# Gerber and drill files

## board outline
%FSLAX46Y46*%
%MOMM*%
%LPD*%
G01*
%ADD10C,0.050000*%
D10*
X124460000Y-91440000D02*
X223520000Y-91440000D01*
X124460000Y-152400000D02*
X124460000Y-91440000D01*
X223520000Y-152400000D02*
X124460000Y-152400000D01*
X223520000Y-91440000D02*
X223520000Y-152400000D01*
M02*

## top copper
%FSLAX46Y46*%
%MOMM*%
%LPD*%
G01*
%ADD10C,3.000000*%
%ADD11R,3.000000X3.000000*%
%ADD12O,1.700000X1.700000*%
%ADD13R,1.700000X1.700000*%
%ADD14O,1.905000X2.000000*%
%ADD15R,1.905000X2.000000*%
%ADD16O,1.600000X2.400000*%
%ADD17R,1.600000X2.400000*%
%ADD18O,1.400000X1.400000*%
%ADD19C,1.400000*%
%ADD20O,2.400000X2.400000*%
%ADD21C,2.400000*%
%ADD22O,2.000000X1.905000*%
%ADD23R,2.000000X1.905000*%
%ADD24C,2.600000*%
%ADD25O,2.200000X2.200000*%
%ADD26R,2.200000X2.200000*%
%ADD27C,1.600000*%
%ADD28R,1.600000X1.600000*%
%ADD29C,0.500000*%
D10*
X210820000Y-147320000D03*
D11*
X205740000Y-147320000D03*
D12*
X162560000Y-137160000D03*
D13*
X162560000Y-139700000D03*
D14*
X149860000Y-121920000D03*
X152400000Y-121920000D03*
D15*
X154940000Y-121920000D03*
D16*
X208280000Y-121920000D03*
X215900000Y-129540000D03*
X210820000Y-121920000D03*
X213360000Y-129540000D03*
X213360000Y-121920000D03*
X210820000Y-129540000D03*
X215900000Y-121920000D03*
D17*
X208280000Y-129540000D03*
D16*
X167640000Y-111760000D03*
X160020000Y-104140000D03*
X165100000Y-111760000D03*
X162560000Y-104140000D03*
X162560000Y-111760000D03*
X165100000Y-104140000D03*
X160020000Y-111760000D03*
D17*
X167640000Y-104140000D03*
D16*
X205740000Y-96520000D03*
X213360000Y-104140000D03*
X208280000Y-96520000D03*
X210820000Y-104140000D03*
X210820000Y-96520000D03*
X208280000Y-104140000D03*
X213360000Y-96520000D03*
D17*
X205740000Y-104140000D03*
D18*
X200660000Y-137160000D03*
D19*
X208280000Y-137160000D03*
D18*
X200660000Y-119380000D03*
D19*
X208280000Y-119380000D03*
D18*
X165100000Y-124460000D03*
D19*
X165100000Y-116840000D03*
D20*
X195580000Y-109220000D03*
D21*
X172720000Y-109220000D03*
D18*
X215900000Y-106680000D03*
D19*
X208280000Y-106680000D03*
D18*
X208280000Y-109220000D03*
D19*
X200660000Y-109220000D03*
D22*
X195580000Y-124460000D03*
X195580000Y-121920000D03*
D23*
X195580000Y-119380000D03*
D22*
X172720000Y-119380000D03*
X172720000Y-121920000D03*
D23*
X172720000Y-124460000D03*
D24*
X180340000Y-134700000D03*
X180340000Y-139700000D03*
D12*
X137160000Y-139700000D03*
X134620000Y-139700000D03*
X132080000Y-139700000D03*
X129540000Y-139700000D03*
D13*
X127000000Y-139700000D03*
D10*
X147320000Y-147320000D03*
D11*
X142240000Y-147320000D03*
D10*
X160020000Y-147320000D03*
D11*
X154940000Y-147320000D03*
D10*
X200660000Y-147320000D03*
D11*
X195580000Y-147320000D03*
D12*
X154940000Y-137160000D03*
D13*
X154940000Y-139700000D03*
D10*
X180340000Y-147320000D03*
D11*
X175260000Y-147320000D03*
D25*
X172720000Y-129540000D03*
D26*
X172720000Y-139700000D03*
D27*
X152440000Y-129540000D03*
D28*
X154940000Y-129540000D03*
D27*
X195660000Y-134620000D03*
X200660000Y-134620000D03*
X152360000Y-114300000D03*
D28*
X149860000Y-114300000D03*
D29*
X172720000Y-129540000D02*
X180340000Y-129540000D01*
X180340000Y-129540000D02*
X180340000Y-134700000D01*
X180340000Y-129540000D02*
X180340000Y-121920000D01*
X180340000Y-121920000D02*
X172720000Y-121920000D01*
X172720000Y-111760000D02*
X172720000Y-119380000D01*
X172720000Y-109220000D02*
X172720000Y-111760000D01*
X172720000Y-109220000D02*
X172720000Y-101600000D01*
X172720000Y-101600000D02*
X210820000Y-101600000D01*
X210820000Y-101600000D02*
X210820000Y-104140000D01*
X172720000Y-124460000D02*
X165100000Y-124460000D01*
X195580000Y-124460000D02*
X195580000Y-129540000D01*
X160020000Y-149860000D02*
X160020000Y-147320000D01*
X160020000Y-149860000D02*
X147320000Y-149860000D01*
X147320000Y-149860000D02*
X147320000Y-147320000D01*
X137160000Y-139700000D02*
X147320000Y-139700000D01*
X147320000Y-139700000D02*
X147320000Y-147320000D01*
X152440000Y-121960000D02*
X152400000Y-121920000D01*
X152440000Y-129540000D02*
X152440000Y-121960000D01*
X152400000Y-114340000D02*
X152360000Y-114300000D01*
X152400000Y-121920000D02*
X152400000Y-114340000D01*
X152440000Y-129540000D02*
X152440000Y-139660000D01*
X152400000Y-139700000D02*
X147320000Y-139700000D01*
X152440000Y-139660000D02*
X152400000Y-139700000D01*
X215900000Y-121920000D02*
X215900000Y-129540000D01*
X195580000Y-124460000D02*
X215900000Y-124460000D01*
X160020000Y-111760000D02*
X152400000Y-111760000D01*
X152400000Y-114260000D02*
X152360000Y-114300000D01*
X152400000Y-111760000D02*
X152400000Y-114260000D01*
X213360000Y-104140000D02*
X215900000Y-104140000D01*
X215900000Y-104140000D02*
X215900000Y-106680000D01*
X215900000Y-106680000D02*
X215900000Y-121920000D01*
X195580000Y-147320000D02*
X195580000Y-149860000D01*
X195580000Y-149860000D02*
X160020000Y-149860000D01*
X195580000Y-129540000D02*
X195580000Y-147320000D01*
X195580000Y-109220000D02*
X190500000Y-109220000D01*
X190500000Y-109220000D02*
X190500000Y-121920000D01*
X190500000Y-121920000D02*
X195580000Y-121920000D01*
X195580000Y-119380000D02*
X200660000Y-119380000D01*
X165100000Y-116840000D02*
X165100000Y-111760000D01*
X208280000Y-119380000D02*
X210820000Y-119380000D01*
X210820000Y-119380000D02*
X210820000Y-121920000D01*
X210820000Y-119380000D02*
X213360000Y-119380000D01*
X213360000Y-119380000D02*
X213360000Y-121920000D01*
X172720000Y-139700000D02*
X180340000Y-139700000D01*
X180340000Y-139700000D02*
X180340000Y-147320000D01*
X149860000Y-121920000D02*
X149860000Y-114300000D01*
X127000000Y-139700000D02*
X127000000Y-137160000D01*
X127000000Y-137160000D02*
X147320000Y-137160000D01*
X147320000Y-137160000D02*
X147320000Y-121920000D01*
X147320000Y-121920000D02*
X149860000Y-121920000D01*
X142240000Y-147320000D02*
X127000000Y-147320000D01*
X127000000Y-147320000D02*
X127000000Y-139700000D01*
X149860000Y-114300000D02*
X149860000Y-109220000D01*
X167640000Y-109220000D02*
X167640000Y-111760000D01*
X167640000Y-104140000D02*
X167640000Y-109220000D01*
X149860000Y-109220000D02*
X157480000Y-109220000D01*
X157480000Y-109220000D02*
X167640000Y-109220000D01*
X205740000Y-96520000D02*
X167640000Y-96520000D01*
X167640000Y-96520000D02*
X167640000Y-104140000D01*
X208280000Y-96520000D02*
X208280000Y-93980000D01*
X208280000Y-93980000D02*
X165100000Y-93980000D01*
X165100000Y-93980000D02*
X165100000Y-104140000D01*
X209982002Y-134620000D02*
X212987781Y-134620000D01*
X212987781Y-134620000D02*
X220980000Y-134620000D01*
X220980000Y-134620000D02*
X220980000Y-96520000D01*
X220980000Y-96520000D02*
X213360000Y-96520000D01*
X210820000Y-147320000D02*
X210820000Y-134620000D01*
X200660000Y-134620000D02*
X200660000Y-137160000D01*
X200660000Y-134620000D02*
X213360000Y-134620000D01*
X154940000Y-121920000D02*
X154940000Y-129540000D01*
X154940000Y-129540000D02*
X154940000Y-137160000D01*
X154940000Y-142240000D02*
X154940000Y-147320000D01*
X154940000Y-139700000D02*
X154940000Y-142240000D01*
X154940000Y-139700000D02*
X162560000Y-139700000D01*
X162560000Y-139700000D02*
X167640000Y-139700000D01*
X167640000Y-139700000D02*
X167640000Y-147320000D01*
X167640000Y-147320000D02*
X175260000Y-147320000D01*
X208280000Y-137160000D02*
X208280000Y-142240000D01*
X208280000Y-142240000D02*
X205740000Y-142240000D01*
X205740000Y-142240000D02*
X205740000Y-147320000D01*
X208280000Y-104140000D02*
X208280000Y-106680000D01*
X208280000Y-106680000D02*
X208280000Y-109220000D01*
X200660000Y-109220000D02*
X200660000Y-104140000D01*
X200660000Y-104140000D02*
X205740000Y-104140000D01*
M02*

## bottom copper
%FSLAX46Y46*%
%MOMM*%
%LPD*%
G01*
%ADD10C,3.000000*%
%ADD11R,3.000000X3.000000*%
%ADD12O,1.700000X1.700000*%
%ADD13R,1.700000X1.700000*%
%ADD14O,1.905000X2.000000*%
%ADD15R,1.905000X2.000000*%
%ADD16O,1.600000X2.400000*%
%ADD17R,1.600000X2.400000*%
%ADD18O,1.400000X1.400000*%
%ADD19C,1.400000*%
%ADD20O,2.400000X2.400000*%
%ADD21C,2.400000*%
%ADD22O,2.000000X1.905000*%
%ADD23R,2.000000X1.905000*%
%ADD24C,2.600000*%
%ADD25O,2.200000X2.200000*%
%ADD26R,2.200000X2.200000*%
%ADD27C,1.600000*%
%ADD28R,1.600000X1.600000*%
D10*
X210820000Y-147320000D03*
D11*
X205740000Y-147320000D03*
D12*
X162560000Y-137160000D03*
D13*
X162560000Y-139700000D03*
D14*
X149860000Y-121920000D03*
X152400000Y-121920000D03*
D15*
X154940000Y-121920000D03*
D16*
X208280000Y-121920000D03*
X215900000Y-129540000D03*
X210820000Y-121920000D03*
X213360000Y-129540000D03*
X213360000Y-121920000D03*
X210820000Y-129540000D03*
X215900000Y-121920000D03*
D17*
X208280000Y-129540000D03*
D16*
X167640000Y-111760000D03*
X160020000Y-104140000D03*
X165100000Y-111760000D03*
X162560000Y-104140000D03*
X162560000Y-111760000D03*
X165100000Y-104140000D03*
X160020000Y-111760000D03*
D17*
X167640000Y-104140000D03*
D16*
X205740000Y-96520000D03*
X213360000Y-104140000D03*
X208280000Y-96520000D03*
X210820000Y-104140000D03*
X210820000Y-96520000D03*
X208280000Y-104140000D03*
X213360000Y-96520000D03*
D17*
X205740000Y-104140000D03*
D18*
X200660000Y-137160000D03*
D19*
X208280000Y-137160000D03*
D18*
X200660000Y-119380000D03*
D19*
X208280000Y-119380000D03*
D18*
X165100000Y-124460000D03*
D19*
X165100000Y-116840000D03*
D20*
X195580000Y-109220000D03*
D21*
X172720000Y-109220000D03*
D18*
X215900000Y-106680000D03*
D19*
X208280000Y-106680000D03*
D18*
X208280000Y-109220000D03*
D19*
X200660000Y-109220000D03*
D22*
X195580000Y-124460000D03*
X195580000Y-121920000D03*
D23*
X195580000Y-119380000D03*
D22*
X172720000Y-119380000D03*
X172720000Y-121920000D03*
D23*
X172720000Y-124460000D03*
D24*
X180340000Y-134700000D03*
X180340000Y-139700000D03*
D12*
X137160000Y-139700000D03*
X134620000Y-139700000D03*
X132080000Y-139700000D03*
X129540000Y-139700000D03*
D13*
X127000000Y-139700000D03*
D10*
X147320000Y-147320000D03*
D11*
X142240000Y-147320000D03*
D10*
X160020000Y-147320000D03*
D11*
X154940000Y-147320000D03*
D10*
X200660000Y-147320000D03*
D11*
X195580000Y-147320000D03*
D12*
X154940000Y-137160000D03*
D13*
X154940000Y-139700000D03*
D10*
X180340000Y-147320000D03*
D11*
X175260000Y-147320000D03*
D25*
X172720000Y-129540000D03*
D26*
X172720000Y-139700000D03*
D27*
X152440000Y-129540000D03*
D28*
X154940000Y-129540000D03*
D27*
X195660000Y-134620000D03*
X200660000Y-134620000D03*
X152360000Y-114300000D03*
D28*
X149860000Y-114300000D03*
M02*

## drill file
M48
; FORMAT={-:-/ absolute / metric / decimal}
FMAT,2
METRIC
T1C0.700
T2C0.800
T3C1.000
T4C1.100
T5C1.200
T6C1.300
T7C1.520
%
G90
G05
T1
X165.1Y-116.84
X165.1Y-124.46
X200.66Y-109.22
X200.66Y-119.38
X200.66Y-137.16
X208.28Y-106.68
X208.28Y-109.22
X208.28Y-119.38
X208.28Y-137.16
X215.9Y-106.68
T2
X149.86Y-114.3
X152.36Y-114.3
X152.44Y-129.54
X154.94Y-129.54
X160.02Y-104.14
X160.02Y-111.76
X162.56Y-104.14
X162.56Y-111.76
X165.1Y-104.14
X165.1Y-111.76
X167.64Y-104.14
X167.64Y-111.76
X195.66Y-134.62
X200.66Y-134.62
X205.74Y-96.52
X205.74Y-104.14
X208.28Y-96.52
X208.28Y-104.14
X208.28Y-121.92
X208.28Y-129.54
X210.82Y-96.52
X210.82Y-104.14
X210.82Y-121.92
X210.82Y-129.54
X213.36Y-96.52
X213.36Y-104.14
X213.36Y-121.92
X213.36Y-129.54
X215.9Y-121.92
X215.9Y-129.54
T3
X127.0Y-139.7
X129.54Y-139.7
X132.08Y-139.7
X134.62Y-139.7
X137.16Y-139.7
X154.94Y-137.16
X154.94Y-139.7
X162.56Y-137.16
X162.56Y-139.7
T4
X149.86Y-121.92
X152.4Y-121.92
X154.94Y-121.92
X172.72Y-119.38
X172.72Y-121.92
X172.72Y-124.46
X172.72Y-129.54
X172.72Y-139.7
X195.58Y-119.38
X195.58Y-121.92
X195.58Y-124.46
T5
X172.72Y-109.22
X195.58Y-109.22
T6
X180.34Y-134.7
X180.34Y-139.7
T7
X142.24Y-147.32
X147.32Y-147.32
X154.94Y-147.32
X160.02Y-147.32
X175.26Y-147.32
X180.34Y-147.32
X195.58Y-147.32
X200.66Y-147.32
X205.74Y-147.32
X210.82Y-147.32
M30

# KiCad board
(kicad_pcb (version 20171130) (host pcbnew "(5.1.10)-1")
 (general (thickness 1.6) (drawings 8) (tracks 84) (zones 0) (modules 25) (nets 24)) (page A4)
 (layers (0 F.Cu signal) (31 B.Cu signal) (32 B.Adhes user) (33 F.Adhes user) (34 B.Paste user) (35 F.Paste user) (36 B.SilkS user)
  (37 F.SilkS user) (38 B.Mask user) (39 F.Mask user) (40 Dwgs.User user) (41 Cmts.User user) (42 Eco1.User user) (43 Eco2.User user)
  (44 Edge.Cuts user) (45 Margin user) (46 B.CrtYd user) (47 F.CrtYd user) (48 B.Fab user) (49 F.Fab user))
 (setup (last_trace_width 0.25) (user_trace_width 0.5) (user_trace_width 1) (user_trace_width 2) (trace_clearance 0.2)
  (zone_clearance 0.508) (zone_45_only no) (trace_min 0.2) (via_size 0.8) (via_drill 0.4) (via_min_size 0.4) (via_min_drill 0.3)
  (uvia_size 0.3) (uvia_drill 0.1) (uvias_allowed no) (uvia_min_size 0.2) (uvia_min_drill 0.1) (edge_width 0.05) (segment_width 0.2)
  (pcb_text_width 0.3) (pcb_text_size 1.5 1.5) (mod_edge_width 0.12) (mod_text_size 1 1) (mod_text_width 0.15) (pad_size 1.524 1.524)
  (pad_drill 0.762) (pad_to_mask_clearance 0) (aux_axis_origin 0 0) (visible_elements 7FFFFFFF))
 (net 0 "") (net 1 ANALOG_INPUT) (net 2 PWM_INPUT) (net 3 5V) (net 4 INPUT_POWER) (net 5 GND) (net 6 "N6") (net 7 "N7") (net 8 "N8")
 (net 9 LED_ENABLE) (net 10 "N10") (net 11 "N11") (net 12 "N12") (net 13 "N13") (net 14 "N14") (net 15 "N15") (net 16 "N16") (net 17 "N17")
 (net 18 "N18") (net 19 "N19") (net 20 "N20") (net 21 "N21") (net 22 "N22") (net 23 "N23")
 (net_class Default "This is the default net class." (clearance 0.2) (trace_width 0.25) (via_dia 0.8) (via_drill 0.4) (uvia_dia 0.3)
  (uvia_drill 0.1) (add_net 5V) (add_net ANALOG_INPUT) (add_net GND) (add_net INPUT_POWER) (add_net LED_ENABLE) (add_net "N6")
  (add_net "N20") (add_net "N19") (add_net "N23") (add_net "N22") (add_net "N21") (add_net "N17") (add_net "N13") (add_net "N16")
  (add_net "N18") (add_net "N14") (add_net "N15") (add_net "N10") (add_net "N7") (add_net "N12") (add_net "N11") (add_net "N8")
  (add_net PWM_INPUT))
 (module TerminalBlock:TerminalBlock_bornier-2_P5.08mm (layer F.Cu) (at 205.74 147.32)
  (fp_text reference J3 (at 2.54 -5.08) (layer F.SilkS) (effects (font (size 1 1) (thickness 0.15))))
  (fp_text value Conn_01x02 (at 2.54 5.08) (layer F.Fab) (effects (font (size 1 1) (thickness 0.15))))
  (pad 2 thru_hole circle (at 5.08 0) (size 3 3) (drill 1.52) (layers *.Cu *.Mask) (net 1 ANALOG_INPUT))
  (pad 1 thru_hole rect (at 0 0) (size 3 3) (drill 1.52) (layers *.Cu *.Mask) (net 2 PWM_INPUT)))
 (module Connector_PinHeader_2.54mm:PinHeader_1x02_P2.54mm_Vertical (layer F.Cu) (at 162.56 139.7 180)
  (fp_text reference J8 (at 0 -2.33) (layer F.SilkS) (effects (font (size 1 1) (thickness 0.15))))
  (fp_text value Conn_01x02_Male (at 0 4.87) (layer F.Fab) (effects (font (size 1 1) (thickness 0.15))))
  (pad 2 thru_hole oval (at 0 2.54 180) (size 1.7 1.7) (drill 1) (layers *.Cu *.Mask) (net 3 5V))
  (pad 1 thru_hole rect (at 0 0 180) (size 1.7 1.7) (drill 1) (layers *.Cu *.Mask) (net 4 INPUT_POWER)))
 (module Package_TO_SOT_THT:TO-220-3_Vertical (layer F.Cu) (at 154.94 121.92 180)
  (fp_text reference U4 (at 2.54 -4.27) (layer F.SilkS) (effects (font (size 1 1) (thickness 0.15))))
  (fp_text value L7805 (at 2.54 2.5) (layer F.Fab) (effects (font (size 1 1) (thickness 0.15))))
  (pad 3 thru_hole oval (at 5.08 0 180) (size 1.905 2) (drill 1.1) (layers *.Cu *.Mask) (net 3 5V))
  (pad 2 thru_hole oval (at 2.54 0 180) (size 1.905 2) (drill 1.1) (layers *.Cu *.Mask) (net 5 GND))
  (pad 1 thru_hole rect (at 0 0 180) (size 1.905 2) (drill 1.1) (layers *.Cu *.Mask) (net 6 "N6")))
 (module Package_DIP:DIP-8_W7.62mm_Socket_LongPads (layer F.Cu) (at 208.28 129.54 90)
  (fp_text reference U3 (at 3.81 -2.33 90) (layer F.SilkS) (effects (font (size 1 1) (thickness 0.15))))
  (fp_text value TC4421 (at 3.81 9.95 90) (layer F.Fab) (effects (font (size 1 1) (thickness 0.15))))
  (pad 8 thru_hole oval (at 7.62 0 90) (size 2.4 1.6) (drill 0.8) (layers *.Cu *.Mask) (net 3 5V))
  (pad 4 thru_hole oval (at 0 7.62 90) (size 2.4 1.6) (drill 0.8) (layers *.Cu *.Mask) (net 5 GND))
  (pad 7 thru_hole oval (at 7.62 2.54 90) (size 2.4 1.6) (drill 0.8) (layers *.Cu *.Mask) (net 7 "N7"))
  (pad 3 thru_hole oval (at 0 5.08 90) (size 2.4 1.6) (drill 0.8) (layers *.Cu *.Mask) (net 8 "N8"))
  (pad 6 thru_hole oval (at 7.62 5.08 90) (size 2.4 1.6) (drill 0.8) (layers *.Cu *.Mask) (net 7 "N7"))
  (pad 2 thru_hole oval (at 0 2.54 90) (size 2.4 1.6) (drill 0.8) (layers *.Cu *.Mask) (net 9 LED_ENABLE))
  (pad 5 thru_hole oval (at 7.62 7.62 90) (size 2.4 1.6) (drill 0.8) (layers *.Cu *.Mask) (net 5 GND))
  (pad 1 thru_hole rect (at 0 0 90) (size 2.4 1.6) (drill 0.8) (layers *.Cu *.Mask) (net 3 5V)))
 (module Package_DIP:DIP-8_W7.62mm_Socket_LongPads (layer F.Cu) (at 167.64 104.14 270)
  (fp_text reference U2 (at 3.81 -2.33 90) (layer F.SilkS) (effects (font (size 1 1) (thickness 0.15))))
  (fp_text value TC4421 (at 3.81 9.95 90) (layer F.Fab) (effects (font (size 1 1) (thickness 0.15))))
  (pad 8 thru_hole oval (at 7.62 0 270) (size 2.4 1.6) (drill 0.8) (layers *.Cu *.Mask) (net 3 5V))
  (pad 4 thru_hole oval (at 0 7.62 270) (size 2.4 1.6) (drill 0.8) (layers *.Cu *.Mask) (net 5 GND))
  (pad 7 thru_hole oval (at 7.62 2.54 270) (size 2.4 1.6) (drill 0.8) (layers *.Cu *.Mask) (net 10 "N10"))
  (pad 3 thru_hole oval (at 0 5.08 270) (size 2.4 1.6) (drill 0.8) (layers *.Cu *.Mask) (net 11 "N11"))
  (pad 6 thru_hole oval (at 7.62 5.08 270) (size 2.4 1.6) (drill 0.8) (layers *.Cu *.Mask) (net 10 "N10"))
  (pad 2 thru_hole oval (at 0 2.54 270) (size 2.4 1.6) (drill 0.8) (layers *.Cu *.Mask) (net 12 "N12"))
  (pad 5 thru_hole oval (at 7.62 7.62 270) (size 2.4 1.6) (drill 0.8) (layers *.Cu *.Mask) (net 5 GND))
  (pad 1 thru_hole rect (at 0 0 270) (size 2.4 1.6) (drill 0.8) (layers *.Cu *.Mask) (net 3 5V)))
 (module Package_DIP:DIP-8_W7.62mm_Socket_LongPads (layer F.Cu) (at 205.74 104.14 90)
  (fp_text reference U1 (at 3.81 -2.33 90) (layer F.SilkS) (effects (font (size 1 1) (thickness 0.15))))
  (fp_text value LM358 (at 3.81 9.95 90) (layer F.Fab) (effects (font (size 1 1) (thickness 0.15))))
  (pad 8 thru_hole oval (at 7.62 0 90) (size 2.4 1.6) (drill 0.8) (layers *.Cu *.Mask) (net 3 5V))
  (pad 4 thru_hole oval (at 0 7.62 90) (size 2.4 1.6) (drill 0.8) (layers *.Cu *.Mask) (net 5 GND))
  (pad 7 thru_hole oval (at 7.62 2.54 90) (size 2.4 1.6) (drill 0.8) (layers *.Cu *.Mask) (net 12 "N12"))
  (pad 3 thru_hole oval (at 0 5.08 90) (size 2.4 1.6) (drill 0.8) (layers *.Cu *.Mask) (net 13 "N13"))
  (pad 6 thru_hole oval (at 7.62 5.08 90) (size 2.4 1.6) (drill 0.8) (layers *.Cu *.Mask) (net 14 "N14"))
  (pad 2 thru_hole oval (at 0 2.54 90) (size 2.4 1.6) (drill 0.8) (layers *.Cu *.Mask) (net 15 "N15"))
  (pad 5 thru_hole oval (at 7.62 7.62 90) (size 2.4 1.6) (drill 0.8) (layers *.Cu *.Mask) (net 1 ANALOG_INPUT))
  (pad 1 thru_hole rect (at 0 0 90) (size 2.4 1.6) (drill 0.8) (layers *.Cu *.Mask) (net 14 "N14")))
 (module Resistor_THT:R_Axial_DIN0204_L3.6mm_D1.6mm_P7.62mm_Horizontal (layer F.Cu) (at 208.28 137.16 180)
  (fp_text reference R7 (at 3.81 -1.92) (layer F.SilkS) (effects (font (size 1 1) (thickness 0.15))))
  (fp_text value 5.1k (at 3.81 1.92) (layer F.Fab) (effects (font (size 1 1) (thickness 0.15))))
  (pad 2 thru_hole oval (at 7.62 0 180) (size 1.4 1.4) (drill 0.7) (layers *.Cu *.Mask) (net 1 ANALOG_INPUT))
  (pad 1 thru_hole circle (at 0 0 180) (size 1.4 1.4) (drill 0.7) (layers *.Cu *.Mask) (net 2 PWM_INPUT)))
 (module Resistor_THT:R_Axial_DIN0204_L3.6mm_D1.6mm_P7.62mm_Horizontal (layer F.Cu) (at 208.28 119.38 180)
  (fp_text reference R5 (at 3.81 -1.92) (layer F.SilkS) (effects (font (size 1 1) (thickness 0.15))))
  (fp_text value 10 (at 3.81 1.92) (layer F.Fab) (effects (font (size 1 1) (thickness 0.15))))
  (pad 2 thru_hole oval (at 7.62 0 180) (size 1.4 1.4) (drill 0.7) (layers *.Cu *.Mask) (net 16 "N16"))
  (pad 1 thru_hole circle (at 0 0 180) (size 1.4 1.4) (drill 0.7) (layers *.Cu *.Mask) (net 7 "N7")))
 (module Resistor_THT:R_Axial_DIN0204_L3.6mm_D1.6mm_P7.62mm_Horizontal (layer F.Cu) (at 165.1 116.84 270)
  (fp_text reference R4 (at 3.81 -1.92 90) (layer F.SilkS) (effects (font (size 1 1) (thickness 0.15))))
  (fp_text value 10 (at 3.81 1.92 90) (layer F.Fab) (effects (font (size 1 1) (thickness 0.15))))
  (pad 2 thru_hole oval (at 7.62 0 270) (size 1.4 1.4) (drill 0.7) (layers *.Cu *.Mask) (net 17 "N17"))
  (pad 1 thru_hole circle (at 0 0 270) (size 1.4 1.4) (drill 0.7) (layers *.Cu *.Mask) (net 10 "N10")))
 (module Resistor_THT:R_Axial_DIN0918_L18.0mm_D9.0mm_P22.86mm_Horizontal (layer F.Cu) (at 172.72 109.22)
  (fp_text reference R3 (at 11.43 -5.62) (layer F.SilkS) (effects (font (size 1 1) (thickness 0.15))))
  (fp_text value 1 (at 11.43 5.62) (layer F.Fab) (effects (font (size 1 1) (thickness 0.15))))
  (pad 2 thru_hole oval (at 22.86 0) (size 2.4 2.4) (drill 1.2) (layers *.Cu *.Mask) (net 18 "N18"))
  (pad 1 thru_hole circle (at 0 0) (size 2.4 2.4) (drill 1.2) (layers *.Cu *.Mask) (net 13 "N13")))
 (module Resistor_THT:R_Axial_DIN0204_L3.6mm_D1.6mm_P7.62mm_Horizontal (layer F.Cu) (at 208.28 106.68)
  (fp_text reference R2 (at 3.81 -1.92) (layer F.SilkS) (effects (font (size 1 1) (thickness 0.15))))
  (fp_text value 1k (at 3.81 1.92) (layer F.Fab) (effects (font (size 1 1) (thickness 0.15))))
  (pad 2 thru_hole oval (at 7.62 0) (size 1.4 1.4) (drill 0.7) (layers *.Cu *.Mask) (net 5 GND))
  (pad 1 thru_hole circle (at 0 0) (size 1.4 1.4) (drill 0.7) (layers *.Cu *.Mask) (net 15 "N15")))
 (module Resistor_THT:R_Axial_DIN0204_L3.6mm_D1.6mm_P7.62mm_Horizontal (layer F.Cu) (at 200.66 109.22)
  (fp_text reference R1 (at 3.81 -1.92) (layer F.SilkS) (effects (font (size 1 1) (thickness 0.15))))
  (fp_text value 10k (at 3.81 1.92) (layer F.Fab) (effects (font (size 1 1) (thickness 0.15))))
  (pad 2 thru_hole oval (at 7.62 0) (size 1.4 1.4) (drill 0.7) (layers *.Cu *.Mask) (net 15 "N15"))
  (pad 1 thru_hole circle (at 0 0) (size 1.4 1.4) (drill 0.7) (layers *.Cu *.Mask) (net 14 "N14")))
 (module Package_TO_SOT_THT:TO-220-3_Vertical (layer F.Cu) (at 195.58 119.38 270)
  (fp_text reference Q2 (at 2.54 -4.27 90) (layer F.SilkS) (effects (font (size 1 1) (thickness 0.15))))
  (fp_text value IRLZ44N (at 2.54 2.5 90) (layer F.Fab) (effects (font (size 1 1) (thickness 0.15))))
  (pad 3 thru_hole oval (at 5.08 0 270) (size 1.905 2) (drill 1.1) (layers *.Cu *.Mask) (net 5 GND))
  (pad 2 thru_hole oval (at 2.54 0 270) (size 1.905 2) (drill 1.1) (layers *.Cu *.Mask) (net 18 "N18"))
  (pad 1 thru_hole rect (at 0 0 270) (size 1.905 2) (drill 1.1) (layers *.Cu *.Mask) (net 16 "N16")))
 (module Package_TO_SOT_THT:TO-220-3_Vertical (layer F.Cu) (at 172.72 124.46 90)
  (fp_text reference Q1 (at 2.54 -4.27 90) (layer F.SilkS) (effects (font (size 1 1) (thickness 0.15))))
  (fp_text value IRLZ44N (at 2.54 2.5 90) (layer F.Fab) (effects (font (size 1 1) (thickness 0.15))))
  (pad 3 thru_hole oval (at 5.08 0 90) (size 1.905 2) (drill 1.1) (layers *.Cu *.Mask) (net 13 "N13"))
  (pad 2 thru_hole oval (at 2.54 0 90) (size 1.905 2) (drill 1.1) (layers *.Cu *.Mask) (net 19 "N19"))
  (pad 1 thru_hole rect (at 0 0 90) (size 1.905 2) (drill 1.1) (layers *.Cu *.Mask) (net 17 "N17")))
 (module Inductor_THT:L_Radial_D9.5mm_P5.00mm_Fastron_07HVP (layer F.Cu) (at 180.34 139.7 90)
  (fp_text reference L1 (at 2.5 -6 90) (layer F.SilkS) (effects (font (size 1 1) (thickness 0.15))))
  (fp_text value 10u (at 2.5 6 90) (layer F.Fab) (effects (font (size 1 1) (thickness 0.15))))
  (pad 2 thru_hole circle (at 5 0 90) (size 2.6 2.6) (drill 1.3) (layers *.Cu *.Mask) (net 19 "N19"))
  (pad 1 thru_hole circle (at 0 0 90) (size 2.6 2.6) (drill 1.3) (layers *.Cu *.Mask) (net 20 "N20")))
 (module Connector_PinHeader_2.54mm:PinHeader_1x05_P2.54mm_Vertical (layer F.Cu) (at 127 139.7 90)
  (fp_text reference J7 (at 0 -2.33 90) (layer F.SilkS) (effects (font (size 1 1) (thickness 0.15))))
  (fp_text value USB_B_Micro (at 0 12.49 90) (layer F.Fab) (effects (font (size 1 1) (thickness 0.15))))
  (pad 5 thru_hole oval (at 0 10.16 90) (size 1.7 1.7) (drill 1) (layers *.Cu *.Mask) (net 5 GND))
  (pad 4 thru_hole oval (at 0 7.62 90) (size 1.7 1.7) (drill 1) (layers *.Cu *.Mask) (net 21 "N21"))
  (pad 3 thru_hole oval (at 0 5.08 90) (size 1.7 1.7) (drill 1) (layers *.Cu *.Mask) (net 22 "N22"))
  (pad 2 thru_hole oval (at 0 2.54 90) (size 1.7 1.7) (drill 1) (layers *.Cu *.Mask) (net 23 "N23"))
  (pad 1 thru_hole rect (at 0 0 90) (size 1.7 1.7) (drill 1) (layers *.Cu *.Mask) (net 3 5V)))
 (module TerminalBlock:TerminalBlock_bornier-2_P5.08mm (layer F.Cu) (at 142.24 147.32)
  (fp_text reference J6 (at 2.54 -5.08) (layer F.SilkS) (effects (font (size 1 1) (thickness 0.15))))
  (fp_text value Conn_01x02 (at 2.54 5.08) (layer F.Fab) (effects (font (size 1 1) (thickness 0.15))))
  (pad 2 thru_hole circle (at 5.08 0) (size 3 3) (drill 1.52) (layers *.Cu *.Mask) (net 5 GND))
  (pad 1 thru_hole rect (at 0 0) (size 3 3) (drill 1.52) (layers *.Cu *.Mask) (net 3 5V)))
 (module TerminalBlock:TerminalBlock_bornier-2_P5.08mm (layer F.Cu) (at 154.94 147.32)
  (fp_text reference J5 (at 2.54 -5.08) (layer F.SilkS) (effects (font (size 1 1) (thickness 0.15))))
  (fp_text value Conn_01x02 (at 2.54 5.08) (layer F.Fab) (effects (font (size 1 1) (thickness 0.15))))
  (pad 2 thru_hole circle (at 5.08 0) (size 3 3) (drill 1.52) (layers *.Cu *.Mask) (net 5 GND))
  (pad 1 thru_hole rect (at 0 0) (size 3 3) (drill 1.52) (layers *.Cu *.Mask) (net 4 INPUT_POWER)))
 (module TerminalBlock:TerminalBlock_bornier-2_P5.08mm (layer F.Cu) (at 195.58 147.32)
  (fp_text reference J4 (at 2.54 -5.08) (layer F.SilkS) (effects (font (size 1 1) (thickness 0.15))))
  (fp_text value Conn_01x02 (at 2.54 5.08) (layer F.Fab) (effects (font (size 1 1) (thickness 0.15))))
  (pad 2 thru_hole circle (at 5.08 0) (size 3 3) (drill 1.52) (layers *.Cu *.Mask) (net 9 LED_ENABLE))
  (pad 1 thru_hole rect (at 0 0) (size 3 3) (drill 1.52) (layers *.Cu *.Mask) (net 5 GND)))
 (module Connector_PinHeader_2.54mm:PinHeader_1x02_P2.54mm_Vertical (layer F.Cu) (at 154.94 139.7 180)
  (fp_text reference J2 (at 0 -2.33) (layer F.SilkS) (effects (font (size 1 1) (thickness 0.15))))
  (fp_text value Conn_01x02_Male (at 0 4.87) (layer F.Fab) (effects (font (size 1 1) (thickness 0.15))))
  (pad 2 thru_hole oval (at 0 2.54 180) (size 1.7 1.7) (drill 1) (layers *.Cu *.Mask) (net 6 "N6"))
  (pad 1 thru_hole rect (at 0 0 180) (size 1.7 1.7) (drill 1) (layers *.Cu *.Mask) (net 4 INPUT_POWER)))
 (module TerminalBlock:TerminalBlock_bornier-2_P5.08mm (layer F.Cu) (at 175.26 147.32)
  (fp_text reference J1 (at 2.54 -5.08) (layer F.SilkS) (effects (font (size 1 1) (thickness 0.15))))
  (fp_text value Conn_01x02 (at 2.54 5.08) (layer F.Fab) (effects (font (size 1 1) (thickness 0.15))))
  (pad 2 thru_hole circle (at 5.08 0) (size 3 3) (drill 1.52) (layers *.Cu *.Mask) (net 20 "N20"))
  (pad 1 thru_hole rect (at 0 0) (size 3 3) (drill 1.52) (layers *.Cu *.Mask) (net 4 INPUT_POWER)))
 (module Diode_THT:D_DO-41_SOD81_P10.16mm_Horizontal (layer F.Cu) (at 172.72 139.7 90)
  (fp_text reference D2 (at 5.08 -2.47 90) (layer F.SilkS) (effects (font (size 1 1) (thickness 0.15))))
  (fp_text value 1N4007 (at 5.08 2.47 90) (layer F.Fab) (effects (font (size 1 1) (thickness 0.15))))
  (pad 2 thru_hole oval (at 10.16 0 90) (size 2.2 2.2) (drill 1.1) (layers *.Cu *.Mask) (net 19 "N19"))
  (pad 1 thru_hole rect (at 0 0 90) (size 2.2 2.2) (drill 1.1) (layers *.Cu *.Mask) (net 20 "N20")))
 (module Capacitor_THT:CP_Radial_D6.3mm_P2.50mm (layer F.Cu) (at 154.94 129.54 180)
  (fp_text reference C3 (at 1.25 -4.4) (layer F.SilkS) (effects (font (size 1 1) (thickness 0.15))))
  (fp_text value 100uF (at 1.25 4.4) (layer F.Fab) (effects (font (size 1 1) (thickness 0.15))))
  (pad 2 thru_hole circle (at 2.5 0 180) (size 1.6 1.6) (drill 0.8) (layers *.Cu *.Mask) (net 5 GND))
  (pad 1 thru_hole rect (at 0 0 180) (size 1.6 1.6) (drill 0.8) (layers *.Cu *.Mask) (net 6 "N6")))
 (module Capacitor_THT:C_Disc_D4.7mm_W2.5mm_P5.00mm (layer F.Cu) (at 200.66 134.62 180)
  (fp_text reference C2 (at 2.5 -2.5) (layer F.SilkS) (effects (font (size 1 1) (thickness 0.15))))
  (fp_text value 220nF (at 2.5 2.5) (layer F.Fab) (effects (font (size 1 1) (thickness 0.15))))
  (pad 2 thru_hole circle (at 5 0 180) (size 1.6 1.6) (drill 0.8) (layers *.Cu *.Mask) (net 5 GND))
  (pad 1 thru_hole circle (at 0 0 180) (size 1.6 1.6) (drill 0.8) (layers *.Cu *.Mask) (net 1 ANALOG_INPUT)))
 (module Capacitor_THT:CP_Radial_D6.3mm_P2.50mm (layer F.Cu) (at 149.86 114.3)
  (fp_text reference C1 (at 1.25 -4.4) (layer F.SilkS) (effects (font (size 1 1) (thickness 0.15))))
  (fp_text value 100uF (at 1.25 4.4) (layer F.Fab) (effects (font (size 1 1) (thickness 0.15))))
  (pad 2 thru_hole circle (at 2.5 0) (size 1.6 1.6) (drill 0.8) (layers *.Cu *.Mask) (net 5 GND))
  (pad 1 thru_hole rect (at 0 0) (size 1.6 1.6) (drill 0.8) (layers *.Cu *.Mask) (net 3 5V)))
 (gr_line (start 124.46 91.44) (end 223.52 91.44) (layer Edge.Cuts) (width 0.05))
 (gr_line (start 124.46 152.4) (end 124.46 91.44) (layer Edge.Cuts) (width 0.05))
 (gr_line (start 223.52 152.4) (end 124.46 152.4) (layer Edge.Cuts) (width 0.05))
 (gr_line (start 223.52 91.44) (end 223.52 152.4) (layer Edge.Cuts) (width 0.05))
 (segment (start 172.72 129.54) (end 180.34 129.54) (width 0.5) (layer F.Cu) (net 19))
 (segment (start 180.34 129.54) (end 180.34 134.7) (width 0.5) (layer F.Cu) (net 19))
 (segment (start 180.34 129.54) (end 180.34 121.92) (width 0.5) (layer F.Cu) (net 19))
 (segment (start 180.34 121.92) (end 172.72 121.92) (width 0.5) (layer F.Cu) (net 19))
 (segment (start 172.72 111.76) (end 172.72 119.38) (width 0.5) (layer F.Cu) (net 13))
 (segment (start 172.72 109.22) (end 172.72 111.76) (width 0.5) (layer F.Cu) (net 13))
 (segment (start 172.72 109.22) (end 172.72 101.6) (width 0.5) (layer F.Cu) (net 13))
 (segment (start 172.72 101.6) (end 210.82 101.6) (width 0.5) (layer F.Cu) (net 13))
 (segment (start 210.82 101.6) (end 210.82 104.14) (width 0.5) (layer F.Cu) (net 13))
 (segment (start 172.72 124.46) (end 165.1 124.46) (width 0.5) (layer F.Cu) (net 17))
 (segment (start 195.58 124.46) (end 195.58 129.54) (width 0.5) (layer F.Cu) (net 5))
 (segment (start 160.02 149.86) (end 160.02 147.32) (width 0.5) (layer F.Cu) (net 5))
 (segment (start 160.02 149.86) (end 147.32 149.86) (width 0.5) (layer F.Cu) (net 5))
 (segment (start 147.32 149.86) (end 147.32 147.32) (width 0.5) (layer F.Cu) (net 5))
 (segment (start 137.16 139.7) (end 147.32 139.7) (width 0.5) (layer F.Cu) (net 5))
 (segment (start 147.32 139.7) (end 147.32 147.32) (width 0.5) (layer F.Cu) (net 5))
 (segment (start 152.44 121.96) (end 152.4 121.92) (width 0.5) (layer F.Cu) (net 5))
 (segment (start 152.44 129.54) (end 152.44 121.96) (width 0.5) (layer F.Cu) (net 5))
 (segment (start 152.4 114.34) (end 152.36 114.3) (width 0.5) (layer F.Cu) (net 5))
 (segment (start 152.4 121.92) (end 152.4 114.34) (width 0.5) (layer F.Cu) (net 5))
 (segment (start 152.44 129.54) (end 152.44 139.66) (width 0.5) (layer F.Cu) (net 5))
 (segment (start 152.4 139.7) (end 147.32 139.7) (width 0.5) (layer F.Cu) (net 5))
 (segment (start 152.44 139.66) (end 152.4 139.7) (width 0.5) (layer F.Cu) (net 5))
 (segment (start 215.9 121.92) (end 215.9 129.54) (width 0.5) (layer F.Cu) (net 5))
 (segment (start 195.58 124.46) (end 215.9 124.46) (width 0.5) (layer F.Cu) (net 5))
 (segment (start 160.02 111.76) (end 152.4 111.76) (width 0.5) (layer F.Cu) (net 5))
 (segment (start 152.4 114.26) (end 152.36 114.3) (width 0.5) (layer F.Cu) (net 5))
 (segment (start 152.4 111.76) (end 152.4 114.26) (width 0.5) (layer F.Cu) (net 5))
 (segment (start 213.36 104.14) (end 215.9 104.14) (width 0.5) (layer F.Cu) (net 5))
 (segment (start 215.9 104.14) (end 215.9 106.68) (width 0.5) (layer F.Cu) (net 5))
 (segment (start 215.9 106.68) (end 215.9 121.92) (width 0.5) (layer F.Cu) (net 5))
 (segment (start 195.58 147.32) (end 195.58 149.86) (width 0.5) (layer F.Cu) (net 5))
 (segment (start 195.58 149.86) (end 160.02 149.86) (width 0.5) (layer F.Cu) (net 5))
 (segment (start 195.58 129.54) (end 195.58 147.32) (width 0.5) (layer F.Cu) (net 5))
 (segment (start 195.58 109.22) (end 190.5 109.22) (width 0.5) (layer F.Cu) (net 18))
 (segment (start 190.5 109.22) (end 190.5 121.92) (width 0.5) (layer F.Cu) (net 18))
 (segment (start 190.5 121.92) (end 195.58 121.92) (width 0.5) (layer F.Cu) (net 18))
 (segment (start 195.58 119.38) (end 200.66 119.38) (width 0.5) (layer F.Cu) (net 16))
 (segment (start 165.1 116.84) (end 165.1 111.76) (width 0.5) (layer F.Cu) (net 10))
 (segment (start 208.28 119.38) (end 210.82 119.38) (width 0.5) (layer F.Cu) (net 7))
 (segment (start 210.82 119.38) (end 210.82 121.92) (width 0.5) (layer F.Cu) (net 7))
 (segment (start 210.82 119.38) (end 213.36 119.38) (width 0.5) (layer F.Cu) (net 7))
 (segment (start 213.36 119.38) (end 213.36 121.92) (width 0.5) (layer F.Cu) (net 7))
 (segment (start 172.72 139.7) (end 180.34 139.7) (width 0.5) (layer F.Cu) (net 20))
 (segment (start 180.34 139.7) (end 180.34 147.32) (width 0.5) (layer F.Cu) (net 20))
 (segment (start 149.86 121.92) (end 149.86 114.3) (width 0.5) (layer F.Cu) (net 3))
 (segment (start 127 139.7) (end 127 137.16) (width 0.5) (layer F.Cu) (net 3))
 (segment (start 127 137.16) (end 147.32 137.16) (width 0.5) (layer F.Cu) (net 3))
 (segment (start 147.32 137.16) (end 147.32 121.92) (width 0.5) (layer F.Cu) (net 3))
 (segment (start 147.32 121.92) (end 149.86 121.92) (width 0.5) (layer F.Cu) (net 3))
 (segment (start 142.24 147.32) (end 127 147.32) (width 0.5) (layer F.Cu) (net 3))
 (segment (start 127 147.32) (end 127 139.7) (width 0.5) (layer F.Cu) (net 3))
 (segment (start 149.86 114.3) (end 149.86 109.22) (width 0.5) (layer F.Cu) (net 3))
 (segment (start 167.64 109.22) (end 167.64 111.76) (width 0.5) (layer F.Cu) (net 3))
 (segment (start 167.64 104.14) (end 167.64 109.22) (width 0.5) (layer F.Cu) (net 3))
 (segment (start 149.86 109.22) (end 157.48 109.22) (width 0.5) (layer F.Cu) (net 3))
 (segment (start 157.48 109.22) (end 167.64 109.22) (width 0.5) (layer F.Cu) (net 3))
 (segment (start 205.74 96.52) (end 167.64 96.52) (width 0.5) (layer F.Cu) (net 3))
 (segment (start 167.64 96.52) (end 167.64 104.14) (width 0.5) (layer F.Cu) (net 3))
 (segment (start 208.28 96.52) (end 208.28 93.98) (width 0.5) (layer F.Cu) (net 12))
 (segment (start 208.28 93.98) (end 165.1 93.98) (width 0.5) (layer F.Cu) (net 12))
 (segment (start 165.1 93.98) (end 165.1 104.14) (width 0.5) (layer F.Cu) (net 12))
 (segment (start 209.982002 134.62) (end 212.987781 134.62) (width 0.5) (layer F.Cu) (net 1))
 (segment (start 212.987781 134.62) (end 220.98 134.62) (width 0.5) (layer F.Cu) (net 1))
 (segment (start 220.98 134.62) (end 220.98 96.52) (width 0.5) (layer F.Cu) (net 1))
 (segment (start 220.98 96.52) (end 213.36 96.52) (width 0.5) (layer F.Cu) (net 1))
 (segment (start 210.82 147.32) (end 210.82 134.62) (width 0.5) (layer F.Cu) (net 1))
 (segment (start 200.66 134.62) (end 200.66 137.16) (width 0.5) (layer F.Cu) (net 1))
 (segment (start 200.66 134.62) (end 213.36 134.62) (width 0.5) (layer F.Cu) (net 1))
 (segment (start 154.94 121.92) (end 154.94 129.54) (width 0.5) (layer F.Cu) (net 6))
 (segment (start 154.94 129.54) (end 154.94 137.16) (width 0.5) (layer F.Cu) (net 6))
 (segment (start 154.94 142.24) (end 154.94 147.32) (width 0.5) (layer F.Cu) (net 4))
 (segment (start 154.94 139.7) (end 154.94 142.24) (width 0.5) (layer F.Cu) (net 4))
 (segment (start 154.94 139.7) (end 162.56 139.7) (width 0.5) (layer F.Cu) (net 4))
 (segment (start 162.56 139.7) (end 167.64 139.7) (width 0.5) (layer F.Cu) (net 4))
 (segment (start 167.64 139.7) (end 167.64 147.32) (width 0.5) (layer F.Cu) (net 4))
 (segment (start 167.64 147.32) (end 175.26 147.32) (width 0.5) (layer F.Cu) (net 4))
 (segment (start 208.28 137.16) (end 208.28 142.24) (width 0.5) (layer F.Cu) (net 2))
 (segment (start 208.28 142.24) (end 205.74 142.24) (width 0.5) (layer F.Cu) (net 2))
 (segment (start 205.74 142.24) (end 205.74 147.32) (width 0.5) (layer F.Cu) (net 2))
 (segment (start 208.28 104.14) (end 208.28 106.68) (width 0.5) (layer F.Cu) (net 15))
 (segment (start 208.28 106.68) (end 208.28 109.22) (width 0.5) (layer F.Cu) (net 15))
 (segment (start 200.66 109.22) (end 200.66 104.14) (width 0.5) (layer F.Cu) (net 14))
 (segment (start 200.66 104.14) (end 205.74 104.14) (width 0.5) (layer F.Cu) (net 14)))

